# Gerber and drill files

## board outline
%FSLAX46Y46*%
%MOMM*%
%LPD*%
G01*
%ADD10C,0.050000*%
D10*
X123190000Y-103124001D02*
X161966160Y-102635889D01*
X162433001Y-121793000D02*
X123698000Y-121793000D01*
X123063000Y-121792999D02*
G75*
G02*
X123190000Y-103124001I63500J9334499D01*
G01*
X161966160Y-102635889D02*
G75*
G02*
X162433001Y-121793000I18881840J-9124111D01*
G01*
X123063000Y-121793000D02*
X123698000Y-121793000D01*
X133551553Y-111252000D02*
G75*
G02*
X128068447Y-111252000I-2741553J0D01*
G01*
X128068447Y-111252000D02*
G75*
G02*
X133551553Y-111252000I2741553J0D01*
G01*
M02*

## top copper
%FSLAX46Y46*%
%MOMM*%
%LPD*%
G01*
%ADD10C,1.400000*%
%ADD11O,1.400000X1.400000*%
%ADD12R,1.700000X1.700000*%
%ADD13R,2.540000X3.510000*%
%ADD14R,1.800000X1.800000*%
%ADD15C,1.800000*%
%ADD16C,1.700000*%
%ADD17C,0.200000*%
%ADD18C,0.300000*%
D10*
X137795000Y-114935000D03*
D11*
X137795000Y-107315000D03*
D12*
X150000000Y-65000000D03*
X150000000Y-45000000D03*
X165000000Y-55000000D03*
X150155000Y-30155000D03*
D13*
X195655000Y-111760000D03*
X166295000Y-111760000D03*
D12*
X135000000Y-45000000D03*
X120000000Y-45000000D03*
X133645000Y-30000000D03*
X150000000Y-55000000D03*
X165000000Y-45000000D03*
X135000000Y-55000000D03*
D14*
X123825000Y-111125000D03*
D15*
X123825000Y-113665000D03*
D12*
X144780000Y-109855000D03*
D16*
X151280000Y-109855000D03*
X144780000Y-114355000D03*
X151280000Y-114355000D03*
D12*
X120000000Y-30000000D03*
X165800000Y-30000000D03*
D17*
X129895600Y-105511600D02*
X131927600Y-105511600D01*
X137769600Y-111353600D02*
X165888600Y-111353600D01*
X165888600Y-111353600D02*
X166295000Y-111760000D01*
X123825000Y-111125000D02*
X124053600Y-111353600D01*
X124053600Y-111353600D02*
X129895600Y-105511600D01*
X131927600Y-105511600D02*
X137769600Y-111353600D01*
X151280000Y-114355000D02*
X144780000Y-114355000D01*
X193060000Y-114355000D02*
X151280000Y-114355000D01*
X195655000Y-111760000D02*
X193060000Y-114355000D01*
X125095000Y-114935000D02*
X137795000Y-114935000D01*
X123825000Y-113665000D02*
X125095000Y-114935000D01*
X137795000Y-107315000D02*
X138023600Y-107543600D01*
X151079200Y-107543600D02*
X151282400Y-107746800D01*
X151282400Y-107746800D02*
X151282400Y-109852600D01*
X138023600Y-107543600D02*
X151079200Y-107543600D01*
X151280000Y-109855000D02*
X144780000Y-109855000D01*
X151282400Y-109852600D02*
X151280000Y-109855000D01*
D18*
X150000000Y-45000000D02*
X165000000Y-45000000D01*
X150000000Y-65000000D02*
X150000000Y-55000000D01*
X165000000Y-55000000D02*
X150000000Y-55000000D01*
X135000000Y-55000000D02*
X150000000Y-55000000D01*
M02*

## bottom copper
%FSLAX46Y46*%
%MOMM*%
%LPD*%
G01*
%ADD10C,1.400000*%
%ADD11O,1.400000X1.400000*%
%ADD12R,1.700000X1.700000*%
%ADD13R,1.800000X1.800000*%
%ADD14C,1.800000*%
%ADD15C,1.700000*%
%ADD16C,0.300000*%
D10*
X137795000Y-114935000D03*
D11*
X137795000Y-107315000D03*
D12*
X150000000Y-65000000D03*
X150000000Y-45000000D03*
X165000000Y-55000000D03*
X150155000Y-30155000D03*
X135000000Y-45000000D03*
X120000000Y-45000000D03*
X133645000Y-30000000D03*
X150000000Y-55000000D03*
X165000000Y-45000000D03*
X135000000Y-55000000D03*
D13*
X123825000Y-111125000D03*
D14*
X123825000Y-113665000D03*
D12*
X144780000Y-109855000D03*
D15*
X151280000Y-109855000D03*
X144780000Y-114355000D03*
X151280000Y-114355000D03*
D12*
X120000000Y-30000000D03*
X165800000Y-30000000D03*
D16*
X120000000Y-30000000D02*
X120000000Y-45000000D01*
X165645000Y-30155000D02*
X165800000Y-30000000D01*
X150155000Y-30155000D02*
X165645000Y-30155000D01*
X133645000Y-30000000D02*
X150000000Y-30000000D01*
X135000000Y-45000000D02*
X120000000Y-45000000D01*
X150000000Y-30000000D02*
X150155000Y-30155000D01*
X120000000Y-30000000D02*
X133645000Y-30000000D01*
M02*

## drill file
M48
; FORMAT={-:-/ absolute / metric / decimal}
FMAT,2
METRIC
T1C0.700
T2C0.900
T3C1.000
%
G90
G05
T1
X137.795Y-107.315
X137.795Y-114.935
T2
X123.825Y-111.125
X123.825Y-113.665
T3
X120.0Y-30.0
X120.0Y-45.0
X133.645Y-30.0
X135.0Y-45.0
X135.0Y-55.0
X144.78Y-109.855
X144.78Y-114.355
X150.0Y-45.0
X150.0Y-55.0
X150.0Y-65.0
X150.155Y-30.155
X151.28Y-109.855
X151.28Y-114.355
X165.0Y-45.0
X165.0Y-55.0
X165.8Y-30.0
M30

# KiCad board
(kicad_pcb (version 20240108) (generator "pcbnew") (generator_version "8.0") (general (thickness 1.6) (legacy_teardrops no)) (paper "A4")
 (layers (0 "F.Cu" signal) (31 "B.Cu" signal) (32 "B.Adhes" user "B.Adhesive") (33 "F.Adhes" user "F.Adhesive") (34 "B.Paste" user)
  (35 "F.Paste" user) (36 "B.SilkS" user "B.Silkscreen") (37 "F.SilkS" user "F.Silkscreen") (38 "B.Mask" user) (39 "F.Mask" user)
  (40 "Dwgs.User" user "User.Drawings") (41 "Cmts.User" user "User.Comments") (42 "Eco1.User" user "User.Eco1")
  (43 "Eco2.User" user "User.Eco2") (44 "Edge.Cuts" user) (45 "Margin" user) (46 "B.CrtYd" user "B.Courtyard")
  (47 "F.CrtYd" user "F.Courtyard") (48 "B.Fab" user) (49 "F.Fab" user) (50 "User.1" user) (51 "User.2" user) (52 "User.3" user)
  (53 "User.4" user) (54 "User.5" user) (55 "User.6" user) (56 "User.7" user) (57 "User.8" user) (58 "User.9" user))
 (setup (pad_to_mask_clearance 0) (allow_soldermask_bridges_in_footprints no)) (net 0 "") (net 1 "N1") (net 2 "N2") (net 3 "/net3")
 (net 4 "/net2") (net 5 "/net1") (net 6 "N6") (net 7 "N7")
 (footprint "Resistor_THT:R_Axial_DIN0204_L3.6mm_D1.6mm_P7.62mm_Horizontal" (layer "F.Cu") (at 137.795 114.935 90)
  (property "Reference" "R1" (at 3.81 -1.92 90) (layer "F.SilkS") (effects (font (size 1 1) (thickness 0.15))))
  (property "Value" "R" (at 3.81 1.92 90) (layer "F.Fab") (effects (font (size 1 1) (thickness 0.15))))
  (pad "1" thru_hole circle (at 0 0 90) (size 1.4 1.4) (drill 0.7) (layers "*.Cu" "*.Mask") (remove_unused_layers no) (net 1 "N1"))
  (pad "2" thru_hole oval (at 7.62 0 90) (size 1.4 1.4) (drill 0.7) (layers "*.Cu" "*.Mask") (remove_unused_layers no) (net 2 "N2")))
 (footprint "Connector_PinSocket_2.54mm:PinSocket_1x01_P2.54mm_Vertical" (layer "F.Cu") (at 150 65)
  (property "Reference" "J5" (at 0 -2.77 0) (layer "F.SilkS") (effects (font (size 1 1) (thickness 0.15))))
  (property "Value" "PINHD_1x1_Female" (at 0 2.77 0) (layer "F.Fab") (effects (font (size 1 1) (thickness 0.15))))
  (pad "1" thru_hole rect (at 0 0) (size 1.7 1.7) (drill 1) (layers "*.Cu" "*.Mask") (remove_unused_layers no) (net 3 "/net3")))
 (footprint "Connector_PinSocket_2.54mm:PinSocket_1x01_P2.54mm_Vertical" (layer "F.Cu") (at 150 45)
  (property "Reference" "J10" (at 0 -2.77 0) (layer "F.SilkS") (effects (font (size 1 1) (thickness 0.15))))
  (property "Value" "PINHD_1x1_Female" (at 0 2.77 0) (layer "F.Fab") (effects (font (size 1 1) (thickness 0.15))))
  (pad "1" thru_hole rect (at 0 0) (size 1.7 1.7) (drill 1) (layers "*.Cu" "*.Mask") (remove_unused_layers no) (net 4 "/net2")))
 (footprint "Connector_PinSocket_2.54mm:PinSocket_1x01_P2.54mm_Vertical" (layer "F.Cu") (at 165 55)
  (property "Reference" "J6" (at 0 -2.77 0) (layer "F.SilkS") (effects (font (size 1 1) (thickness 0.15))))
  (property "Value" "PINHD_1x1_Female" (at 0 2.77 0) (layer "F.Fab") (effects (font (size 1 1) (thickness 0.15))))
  (pad "1" thru_hole rect (at 0 0) (size 1.7 1.7) (drill 1) (layers "*.Cu" "*.Mask") (remove_unused_layers no) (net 3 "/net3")))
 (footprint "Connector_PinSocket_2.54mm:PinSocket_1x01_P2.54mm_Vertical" (layer "F.Cu") (at 150.155 30.155)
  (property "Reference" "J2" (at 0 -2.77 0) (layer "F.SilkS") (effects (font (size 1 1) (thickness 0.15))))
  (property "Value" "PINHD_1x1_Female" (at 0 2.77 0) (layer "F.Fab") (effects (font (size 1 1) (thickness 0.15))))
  (pad "1" thru_hole rect (at 0 0) (size 1.7 1.7) (drill 1) (layers "*.Cu" "*.Mask") (remove_unused_layers no) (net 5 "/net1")))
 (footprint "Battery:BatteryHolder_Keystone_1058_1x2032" (layer "F.Cu") (at 180.975 111.76 180)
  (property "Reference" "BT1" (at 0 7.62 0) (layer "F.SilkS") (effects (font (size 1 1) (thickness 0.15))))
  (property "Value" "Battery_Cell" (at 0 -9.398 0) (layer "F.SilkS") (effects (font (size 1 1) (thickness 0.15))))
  (pad "1" smd rect (at -14.68 0 180) (size 2.54 3.51) (layers "F.Cu" "F.Paste" "F.Mask") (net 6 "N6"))
  (pad "2" smd rect (at 14.68 0 180) (size 2.54 3.51) (layers "F.Cu" "F.Paste" "F.Mask") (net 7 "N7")))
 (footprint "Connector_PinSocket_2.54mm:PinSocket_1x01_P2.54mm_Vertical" (layer "F.Cu") (at 135 45)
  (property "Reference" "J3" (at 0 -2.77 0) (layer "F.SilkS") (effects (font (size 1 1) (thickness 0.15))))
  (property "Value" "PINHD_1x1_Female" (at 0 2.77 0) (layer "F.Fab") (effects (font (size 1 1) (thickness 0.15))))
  (pad "1" thru_hole rect (at 0 0) (size 1.7 1.7) (drill 1) (layers "*.Cu" "*.Mask") (remove_unused_layers no) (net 5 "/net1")))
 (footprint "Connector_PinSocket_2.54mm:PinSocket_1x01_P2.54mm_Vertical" (layer "F.Cu") (at 120 45)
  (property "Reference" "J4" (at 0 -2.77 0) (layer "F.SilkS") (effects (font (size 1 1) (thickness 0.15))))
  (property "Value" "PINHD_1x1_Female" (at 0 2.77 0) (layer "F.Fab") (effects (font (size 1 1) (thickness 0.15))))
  (pad "1" thru_hole rect (at 0 0) (size 1.7 1.7) (drill 1) (layers "*.Cu" "*.Mask") (remove_unused_layers no) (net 5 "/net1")))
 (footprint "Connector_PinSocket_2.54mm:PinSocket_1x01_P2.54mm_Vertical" (layer "F.Cu") (at 133.645 30)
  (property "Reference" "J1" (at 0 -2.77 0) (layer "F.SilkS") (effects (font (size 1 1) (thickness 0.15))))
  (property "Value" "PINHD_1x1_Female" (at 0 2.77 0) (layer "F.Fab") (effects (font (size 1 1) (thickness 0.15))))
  (pad "1" thru_hole rect (at 0 0) (size 1.7 1.7) (drill 1) (layers "*.Cu" "*.Mask") (remove_unused_layers no) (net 5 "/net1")))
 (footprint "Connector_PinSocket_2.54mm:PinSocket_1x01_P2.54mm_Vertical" (layer "F.Cu") (at 150 55)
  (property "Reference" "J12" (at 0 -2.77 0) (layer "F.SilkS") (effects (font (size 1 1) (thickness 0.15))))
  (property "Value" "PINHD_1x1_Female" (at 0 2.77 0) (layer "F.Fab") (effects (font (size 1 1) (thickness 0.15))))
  (pad "1" thru_hole rect (at 0 0) (size 1.7 1.7) (drill 1) (layers "*.Cu" "*.Mask") (remove_unused_layers no) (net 3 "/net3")))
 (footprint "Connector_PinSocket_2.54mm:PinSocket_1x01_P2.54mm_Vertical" (layer "F.Cu") (at 165 45)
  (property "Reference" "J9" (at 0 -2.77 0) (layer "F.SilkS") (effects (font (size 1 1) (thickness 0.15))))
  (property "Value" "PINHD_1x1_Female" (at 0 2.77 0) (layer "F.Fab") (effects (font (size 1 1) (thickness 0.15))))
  (pad "1" thru_hole rect (at 0 0) (size 1.7 1.7) (drill 1) (layers "*.Cu" "*.Mask") (remove_unused_layers no) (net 4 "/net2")))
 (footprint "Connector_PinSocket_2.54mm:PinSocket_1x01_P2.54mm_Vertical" (layer "F.Cu") (at 135 55)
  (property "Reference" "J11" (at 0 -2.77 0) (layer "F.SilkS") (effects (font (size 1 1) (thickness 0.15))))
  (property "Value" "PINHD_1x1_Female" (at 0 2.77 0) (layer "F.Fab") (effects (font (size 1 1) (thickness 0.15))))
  (pad "1" thru_hole rect (at 0 0) (size 1.7 1.7) (drill 1) (layers "*.Cu" "*.Mask") (remove_unused_layers no) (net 3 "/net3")))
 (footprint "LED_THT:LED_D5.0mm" (layer "F.Cu") (at 123.825 111.125 -90)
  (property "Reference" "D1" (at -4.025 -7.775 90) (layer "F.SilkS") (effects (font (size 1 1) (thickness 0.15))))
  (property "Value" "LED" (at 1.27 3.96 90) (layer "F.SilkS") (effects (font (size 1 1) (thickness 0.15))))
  (pad "1" thru_hole rect (at 0 0 270) (size 1.8 1.8) (drill 0.9) (layers "*.Cu" "*.Mask") (remove_unused_layers no) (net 7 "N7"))
  (pad "2" thru_hole circle (at 2.54 0 270) (size 1.8 1.8) (drill 0.9) (layers "*.Cu" "*.Mask") (remove_unused_layers no) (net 1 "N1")))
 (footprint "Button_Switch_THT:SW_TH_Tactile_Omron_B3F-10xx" (layer "F.Cu") (at 144.78 109.855)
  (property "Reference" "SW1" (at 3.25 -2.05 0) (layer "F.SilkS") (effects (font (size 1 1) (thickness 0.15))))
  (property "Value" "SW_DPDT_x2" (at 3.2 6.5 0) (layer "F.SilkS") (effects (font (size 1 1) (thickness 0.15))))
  (pad "1" thru_hole rect (at 0 0) (size 1.7 1.7) (drill 1) (layers "*.Cu" "*.Mask") (remove_unused_layers no) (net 2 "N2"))
  (pad "1" thru_hole circle (at 6.5 0) (size 1.7 1.7) (drill 1) (layers "*.Cu" "*.Mask") (remove_unused_layers no) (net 2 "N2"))
  (pad "2" thru_hole circle (at 0 4.5) (size 1.7 1.7) (drill 1) (layers "*.Cu" "*.Mask") (remove_unused_layers no) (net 6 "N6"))
  (pad "2" thru_hole circle (at 6.5 4.5) (size 1.7 1.7) (drill 1) (layers "*.Cu" "*.Mask") (remove_unused_layers no) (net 6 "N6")))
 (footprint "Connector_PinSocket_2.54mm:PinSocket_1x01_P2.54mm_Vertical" (layer "F.Cu") (at 120 30)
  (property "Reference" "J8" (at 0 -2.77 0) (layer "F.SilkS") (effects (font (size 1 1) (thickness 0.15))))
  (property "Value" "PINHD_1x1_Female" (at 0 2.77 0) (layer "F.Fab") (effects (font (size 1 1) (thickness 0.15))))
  (pad "1" thru_hole rect (at 0 0) (size 1.7 1.7) (drill 1) (layers "*.Cu" "*.Mask") (remove_unused_layers no) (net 5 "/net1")))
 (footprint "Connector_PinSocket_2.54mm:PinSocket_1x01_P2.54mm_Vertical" (layer "F.Cu") (at 165.8 30)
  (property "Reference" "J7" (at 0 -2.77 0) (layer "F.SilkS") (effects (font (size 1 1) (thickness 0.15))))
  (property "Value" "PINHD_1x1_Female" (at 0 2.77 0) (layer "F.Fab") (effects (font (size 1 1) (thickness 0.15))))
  (pad "1" thru_hole rect (at 0 0) (size 1.7 1.7) (drill 1) (layers "*.Cu" "*.Mask") (remove_unused_layers no) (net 5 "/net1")))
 (gr_line (start 123.19 103.124001) (end 161.96616 102.635889) (locked yes) (stroke (width 0.05) (type default)) (layer "Edge.Cuts"))
 (gr_line (start 162.433001 121.793) (end 123.698 121.793) (locked yes) (stroke (width 0.05) (type default)) (layer "Edge.Cuts"))
 (gr_arc (start 123.063 121.792999) (mid 113.792001 112.395) (end 123.19 103.124001) (locked yes) (stroke (width 0.05) (type default))
  (layer "Edge.Cuts"))
 (gr_arc (start 161.96616 102.635889) (mid 201.812548 111.249114) (end 162.433001 121.793) (locked yes) (stroke (width 0.05) (type default))
  (layer "Edge.Cuts"))
 (gr_line (start 123.063 121.793) (end 123.698 121.793) (locked yes) (stroke (width 0.05) (type default)) (layer "Edge.Cuts"))
 (gr_circle (center 130.81 111.252) (end 133.477 111.887) (locked yes) (stroke (width 0.05) (type default)) (fill none) (layer "Edge.Cuts"))
 (segment (start 129.8956 105.5116) (end 131.9276 105.5116) (width 0.2) (layer "F.Cu") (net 7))
 (segment (start 137.7696 111.3536) (end 165.8886 111.3536) (width 0.2) (layer "F.Cu") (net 7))
 (segment (start 165.8886 111.3536) (end 166.295 111.76) (width 0.2) (layer "F.Cu") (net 7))
 (segment (start 123.825 111.125) (end 124.0536 111.3536) (width 0.2) (layer "F.Cu") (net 7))
 (segment (start 124.0536 111.3536) (end 129.8956 105.5116) (width 0.2) (layer "F.Cu") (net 7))
 (segment (start 131.9276 105.5116) (end 137.7696 111.3536) (width 0.2) (layer "F.Cu") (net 7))
 (segment (start 151.28 114.355) (end 144.78 114.355) (width 0.2) (layer "F.Cu") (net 6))
 (segment (start 193.06 114.355) (end 151.28 114.355) (width 0.2) (layer "F.Cu") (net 6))
 (segment (start 195.655 111.76) (end 193.06 114.355) (width 0.2) (layer "F.Cu") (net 6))
 (segment (start 125.095 114.935) (end 137.795 114.935) (width 0.2) (layer "F.Cu") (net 1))
 (segment (start 123.825 113.665) (end 125.095 114.935) (width 0.2) (layer "F.Cu") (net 1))
 (segment (start 137.795 107.315) (end 138.0236 107.5436) (width 0.2) (layer "F.Cu") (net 2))
 (segment (start 151.0792 107.5436) (end 151.2824 107.7468) (width 0.2) (layer "F.Cu") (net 2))
 (segment (start 151.2824 107.7468) (end 151.2824 109.8526) (width 0.2) (layer "F.Cu") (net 2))
 (segment (start 138.0236 107.5436) (end 151.0792 107.5436) (width 0.2) (layer "F.Cu") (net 2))
 (segment (start 151.28 109.855) (end 144.78 109.855) (width 0.2) (layer "F.Cu") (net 2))
 (segment (start 151.2824 109.8526) (end 151.28 109.855) (width 0.2) (layer "F.Cu") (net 2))
 (segment (start 120 30) (end 120 45) (width 0.3) (layer "B.Cu") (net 5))
 (segment (start 165.645 30.155) (end 165.8 30) (width 0.3) (layer "B.Cu") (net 5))
 (segment (start 150.155 30.155) (end 165.645 30.155) (width 0.3) (layer "B.Cu") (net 5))
 (segment (start 133.645 30) (end 150 30) (width 0.3) (layer "B.Cu") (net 5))
 (segment (start 135 45) (end 120 45) (width 0.3) (layer "B.Cu") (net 5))
 (segment (start 150 30) (end 150.155 30.155) (width 0.3) (layer "B.Cu") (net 5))
 (segment (start 120 30) (end 133.645 30) (width 0.3) (layer "B.Cu") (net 5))
 (segment (start 150 45) (end 165 45) (width 0.3) (layer "F.Cu") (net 4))
 (segment (start 150 65) (end 150 55) (width 0.3) (layer "F.Cu") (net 3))
 (segment (start 165 55) (end 150 55) (width 0.3) (layer "F.Cu") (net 3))
 (segment (start 135 55) (end 150 55) (width 0.3) (layer "F.Cu") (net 3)))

